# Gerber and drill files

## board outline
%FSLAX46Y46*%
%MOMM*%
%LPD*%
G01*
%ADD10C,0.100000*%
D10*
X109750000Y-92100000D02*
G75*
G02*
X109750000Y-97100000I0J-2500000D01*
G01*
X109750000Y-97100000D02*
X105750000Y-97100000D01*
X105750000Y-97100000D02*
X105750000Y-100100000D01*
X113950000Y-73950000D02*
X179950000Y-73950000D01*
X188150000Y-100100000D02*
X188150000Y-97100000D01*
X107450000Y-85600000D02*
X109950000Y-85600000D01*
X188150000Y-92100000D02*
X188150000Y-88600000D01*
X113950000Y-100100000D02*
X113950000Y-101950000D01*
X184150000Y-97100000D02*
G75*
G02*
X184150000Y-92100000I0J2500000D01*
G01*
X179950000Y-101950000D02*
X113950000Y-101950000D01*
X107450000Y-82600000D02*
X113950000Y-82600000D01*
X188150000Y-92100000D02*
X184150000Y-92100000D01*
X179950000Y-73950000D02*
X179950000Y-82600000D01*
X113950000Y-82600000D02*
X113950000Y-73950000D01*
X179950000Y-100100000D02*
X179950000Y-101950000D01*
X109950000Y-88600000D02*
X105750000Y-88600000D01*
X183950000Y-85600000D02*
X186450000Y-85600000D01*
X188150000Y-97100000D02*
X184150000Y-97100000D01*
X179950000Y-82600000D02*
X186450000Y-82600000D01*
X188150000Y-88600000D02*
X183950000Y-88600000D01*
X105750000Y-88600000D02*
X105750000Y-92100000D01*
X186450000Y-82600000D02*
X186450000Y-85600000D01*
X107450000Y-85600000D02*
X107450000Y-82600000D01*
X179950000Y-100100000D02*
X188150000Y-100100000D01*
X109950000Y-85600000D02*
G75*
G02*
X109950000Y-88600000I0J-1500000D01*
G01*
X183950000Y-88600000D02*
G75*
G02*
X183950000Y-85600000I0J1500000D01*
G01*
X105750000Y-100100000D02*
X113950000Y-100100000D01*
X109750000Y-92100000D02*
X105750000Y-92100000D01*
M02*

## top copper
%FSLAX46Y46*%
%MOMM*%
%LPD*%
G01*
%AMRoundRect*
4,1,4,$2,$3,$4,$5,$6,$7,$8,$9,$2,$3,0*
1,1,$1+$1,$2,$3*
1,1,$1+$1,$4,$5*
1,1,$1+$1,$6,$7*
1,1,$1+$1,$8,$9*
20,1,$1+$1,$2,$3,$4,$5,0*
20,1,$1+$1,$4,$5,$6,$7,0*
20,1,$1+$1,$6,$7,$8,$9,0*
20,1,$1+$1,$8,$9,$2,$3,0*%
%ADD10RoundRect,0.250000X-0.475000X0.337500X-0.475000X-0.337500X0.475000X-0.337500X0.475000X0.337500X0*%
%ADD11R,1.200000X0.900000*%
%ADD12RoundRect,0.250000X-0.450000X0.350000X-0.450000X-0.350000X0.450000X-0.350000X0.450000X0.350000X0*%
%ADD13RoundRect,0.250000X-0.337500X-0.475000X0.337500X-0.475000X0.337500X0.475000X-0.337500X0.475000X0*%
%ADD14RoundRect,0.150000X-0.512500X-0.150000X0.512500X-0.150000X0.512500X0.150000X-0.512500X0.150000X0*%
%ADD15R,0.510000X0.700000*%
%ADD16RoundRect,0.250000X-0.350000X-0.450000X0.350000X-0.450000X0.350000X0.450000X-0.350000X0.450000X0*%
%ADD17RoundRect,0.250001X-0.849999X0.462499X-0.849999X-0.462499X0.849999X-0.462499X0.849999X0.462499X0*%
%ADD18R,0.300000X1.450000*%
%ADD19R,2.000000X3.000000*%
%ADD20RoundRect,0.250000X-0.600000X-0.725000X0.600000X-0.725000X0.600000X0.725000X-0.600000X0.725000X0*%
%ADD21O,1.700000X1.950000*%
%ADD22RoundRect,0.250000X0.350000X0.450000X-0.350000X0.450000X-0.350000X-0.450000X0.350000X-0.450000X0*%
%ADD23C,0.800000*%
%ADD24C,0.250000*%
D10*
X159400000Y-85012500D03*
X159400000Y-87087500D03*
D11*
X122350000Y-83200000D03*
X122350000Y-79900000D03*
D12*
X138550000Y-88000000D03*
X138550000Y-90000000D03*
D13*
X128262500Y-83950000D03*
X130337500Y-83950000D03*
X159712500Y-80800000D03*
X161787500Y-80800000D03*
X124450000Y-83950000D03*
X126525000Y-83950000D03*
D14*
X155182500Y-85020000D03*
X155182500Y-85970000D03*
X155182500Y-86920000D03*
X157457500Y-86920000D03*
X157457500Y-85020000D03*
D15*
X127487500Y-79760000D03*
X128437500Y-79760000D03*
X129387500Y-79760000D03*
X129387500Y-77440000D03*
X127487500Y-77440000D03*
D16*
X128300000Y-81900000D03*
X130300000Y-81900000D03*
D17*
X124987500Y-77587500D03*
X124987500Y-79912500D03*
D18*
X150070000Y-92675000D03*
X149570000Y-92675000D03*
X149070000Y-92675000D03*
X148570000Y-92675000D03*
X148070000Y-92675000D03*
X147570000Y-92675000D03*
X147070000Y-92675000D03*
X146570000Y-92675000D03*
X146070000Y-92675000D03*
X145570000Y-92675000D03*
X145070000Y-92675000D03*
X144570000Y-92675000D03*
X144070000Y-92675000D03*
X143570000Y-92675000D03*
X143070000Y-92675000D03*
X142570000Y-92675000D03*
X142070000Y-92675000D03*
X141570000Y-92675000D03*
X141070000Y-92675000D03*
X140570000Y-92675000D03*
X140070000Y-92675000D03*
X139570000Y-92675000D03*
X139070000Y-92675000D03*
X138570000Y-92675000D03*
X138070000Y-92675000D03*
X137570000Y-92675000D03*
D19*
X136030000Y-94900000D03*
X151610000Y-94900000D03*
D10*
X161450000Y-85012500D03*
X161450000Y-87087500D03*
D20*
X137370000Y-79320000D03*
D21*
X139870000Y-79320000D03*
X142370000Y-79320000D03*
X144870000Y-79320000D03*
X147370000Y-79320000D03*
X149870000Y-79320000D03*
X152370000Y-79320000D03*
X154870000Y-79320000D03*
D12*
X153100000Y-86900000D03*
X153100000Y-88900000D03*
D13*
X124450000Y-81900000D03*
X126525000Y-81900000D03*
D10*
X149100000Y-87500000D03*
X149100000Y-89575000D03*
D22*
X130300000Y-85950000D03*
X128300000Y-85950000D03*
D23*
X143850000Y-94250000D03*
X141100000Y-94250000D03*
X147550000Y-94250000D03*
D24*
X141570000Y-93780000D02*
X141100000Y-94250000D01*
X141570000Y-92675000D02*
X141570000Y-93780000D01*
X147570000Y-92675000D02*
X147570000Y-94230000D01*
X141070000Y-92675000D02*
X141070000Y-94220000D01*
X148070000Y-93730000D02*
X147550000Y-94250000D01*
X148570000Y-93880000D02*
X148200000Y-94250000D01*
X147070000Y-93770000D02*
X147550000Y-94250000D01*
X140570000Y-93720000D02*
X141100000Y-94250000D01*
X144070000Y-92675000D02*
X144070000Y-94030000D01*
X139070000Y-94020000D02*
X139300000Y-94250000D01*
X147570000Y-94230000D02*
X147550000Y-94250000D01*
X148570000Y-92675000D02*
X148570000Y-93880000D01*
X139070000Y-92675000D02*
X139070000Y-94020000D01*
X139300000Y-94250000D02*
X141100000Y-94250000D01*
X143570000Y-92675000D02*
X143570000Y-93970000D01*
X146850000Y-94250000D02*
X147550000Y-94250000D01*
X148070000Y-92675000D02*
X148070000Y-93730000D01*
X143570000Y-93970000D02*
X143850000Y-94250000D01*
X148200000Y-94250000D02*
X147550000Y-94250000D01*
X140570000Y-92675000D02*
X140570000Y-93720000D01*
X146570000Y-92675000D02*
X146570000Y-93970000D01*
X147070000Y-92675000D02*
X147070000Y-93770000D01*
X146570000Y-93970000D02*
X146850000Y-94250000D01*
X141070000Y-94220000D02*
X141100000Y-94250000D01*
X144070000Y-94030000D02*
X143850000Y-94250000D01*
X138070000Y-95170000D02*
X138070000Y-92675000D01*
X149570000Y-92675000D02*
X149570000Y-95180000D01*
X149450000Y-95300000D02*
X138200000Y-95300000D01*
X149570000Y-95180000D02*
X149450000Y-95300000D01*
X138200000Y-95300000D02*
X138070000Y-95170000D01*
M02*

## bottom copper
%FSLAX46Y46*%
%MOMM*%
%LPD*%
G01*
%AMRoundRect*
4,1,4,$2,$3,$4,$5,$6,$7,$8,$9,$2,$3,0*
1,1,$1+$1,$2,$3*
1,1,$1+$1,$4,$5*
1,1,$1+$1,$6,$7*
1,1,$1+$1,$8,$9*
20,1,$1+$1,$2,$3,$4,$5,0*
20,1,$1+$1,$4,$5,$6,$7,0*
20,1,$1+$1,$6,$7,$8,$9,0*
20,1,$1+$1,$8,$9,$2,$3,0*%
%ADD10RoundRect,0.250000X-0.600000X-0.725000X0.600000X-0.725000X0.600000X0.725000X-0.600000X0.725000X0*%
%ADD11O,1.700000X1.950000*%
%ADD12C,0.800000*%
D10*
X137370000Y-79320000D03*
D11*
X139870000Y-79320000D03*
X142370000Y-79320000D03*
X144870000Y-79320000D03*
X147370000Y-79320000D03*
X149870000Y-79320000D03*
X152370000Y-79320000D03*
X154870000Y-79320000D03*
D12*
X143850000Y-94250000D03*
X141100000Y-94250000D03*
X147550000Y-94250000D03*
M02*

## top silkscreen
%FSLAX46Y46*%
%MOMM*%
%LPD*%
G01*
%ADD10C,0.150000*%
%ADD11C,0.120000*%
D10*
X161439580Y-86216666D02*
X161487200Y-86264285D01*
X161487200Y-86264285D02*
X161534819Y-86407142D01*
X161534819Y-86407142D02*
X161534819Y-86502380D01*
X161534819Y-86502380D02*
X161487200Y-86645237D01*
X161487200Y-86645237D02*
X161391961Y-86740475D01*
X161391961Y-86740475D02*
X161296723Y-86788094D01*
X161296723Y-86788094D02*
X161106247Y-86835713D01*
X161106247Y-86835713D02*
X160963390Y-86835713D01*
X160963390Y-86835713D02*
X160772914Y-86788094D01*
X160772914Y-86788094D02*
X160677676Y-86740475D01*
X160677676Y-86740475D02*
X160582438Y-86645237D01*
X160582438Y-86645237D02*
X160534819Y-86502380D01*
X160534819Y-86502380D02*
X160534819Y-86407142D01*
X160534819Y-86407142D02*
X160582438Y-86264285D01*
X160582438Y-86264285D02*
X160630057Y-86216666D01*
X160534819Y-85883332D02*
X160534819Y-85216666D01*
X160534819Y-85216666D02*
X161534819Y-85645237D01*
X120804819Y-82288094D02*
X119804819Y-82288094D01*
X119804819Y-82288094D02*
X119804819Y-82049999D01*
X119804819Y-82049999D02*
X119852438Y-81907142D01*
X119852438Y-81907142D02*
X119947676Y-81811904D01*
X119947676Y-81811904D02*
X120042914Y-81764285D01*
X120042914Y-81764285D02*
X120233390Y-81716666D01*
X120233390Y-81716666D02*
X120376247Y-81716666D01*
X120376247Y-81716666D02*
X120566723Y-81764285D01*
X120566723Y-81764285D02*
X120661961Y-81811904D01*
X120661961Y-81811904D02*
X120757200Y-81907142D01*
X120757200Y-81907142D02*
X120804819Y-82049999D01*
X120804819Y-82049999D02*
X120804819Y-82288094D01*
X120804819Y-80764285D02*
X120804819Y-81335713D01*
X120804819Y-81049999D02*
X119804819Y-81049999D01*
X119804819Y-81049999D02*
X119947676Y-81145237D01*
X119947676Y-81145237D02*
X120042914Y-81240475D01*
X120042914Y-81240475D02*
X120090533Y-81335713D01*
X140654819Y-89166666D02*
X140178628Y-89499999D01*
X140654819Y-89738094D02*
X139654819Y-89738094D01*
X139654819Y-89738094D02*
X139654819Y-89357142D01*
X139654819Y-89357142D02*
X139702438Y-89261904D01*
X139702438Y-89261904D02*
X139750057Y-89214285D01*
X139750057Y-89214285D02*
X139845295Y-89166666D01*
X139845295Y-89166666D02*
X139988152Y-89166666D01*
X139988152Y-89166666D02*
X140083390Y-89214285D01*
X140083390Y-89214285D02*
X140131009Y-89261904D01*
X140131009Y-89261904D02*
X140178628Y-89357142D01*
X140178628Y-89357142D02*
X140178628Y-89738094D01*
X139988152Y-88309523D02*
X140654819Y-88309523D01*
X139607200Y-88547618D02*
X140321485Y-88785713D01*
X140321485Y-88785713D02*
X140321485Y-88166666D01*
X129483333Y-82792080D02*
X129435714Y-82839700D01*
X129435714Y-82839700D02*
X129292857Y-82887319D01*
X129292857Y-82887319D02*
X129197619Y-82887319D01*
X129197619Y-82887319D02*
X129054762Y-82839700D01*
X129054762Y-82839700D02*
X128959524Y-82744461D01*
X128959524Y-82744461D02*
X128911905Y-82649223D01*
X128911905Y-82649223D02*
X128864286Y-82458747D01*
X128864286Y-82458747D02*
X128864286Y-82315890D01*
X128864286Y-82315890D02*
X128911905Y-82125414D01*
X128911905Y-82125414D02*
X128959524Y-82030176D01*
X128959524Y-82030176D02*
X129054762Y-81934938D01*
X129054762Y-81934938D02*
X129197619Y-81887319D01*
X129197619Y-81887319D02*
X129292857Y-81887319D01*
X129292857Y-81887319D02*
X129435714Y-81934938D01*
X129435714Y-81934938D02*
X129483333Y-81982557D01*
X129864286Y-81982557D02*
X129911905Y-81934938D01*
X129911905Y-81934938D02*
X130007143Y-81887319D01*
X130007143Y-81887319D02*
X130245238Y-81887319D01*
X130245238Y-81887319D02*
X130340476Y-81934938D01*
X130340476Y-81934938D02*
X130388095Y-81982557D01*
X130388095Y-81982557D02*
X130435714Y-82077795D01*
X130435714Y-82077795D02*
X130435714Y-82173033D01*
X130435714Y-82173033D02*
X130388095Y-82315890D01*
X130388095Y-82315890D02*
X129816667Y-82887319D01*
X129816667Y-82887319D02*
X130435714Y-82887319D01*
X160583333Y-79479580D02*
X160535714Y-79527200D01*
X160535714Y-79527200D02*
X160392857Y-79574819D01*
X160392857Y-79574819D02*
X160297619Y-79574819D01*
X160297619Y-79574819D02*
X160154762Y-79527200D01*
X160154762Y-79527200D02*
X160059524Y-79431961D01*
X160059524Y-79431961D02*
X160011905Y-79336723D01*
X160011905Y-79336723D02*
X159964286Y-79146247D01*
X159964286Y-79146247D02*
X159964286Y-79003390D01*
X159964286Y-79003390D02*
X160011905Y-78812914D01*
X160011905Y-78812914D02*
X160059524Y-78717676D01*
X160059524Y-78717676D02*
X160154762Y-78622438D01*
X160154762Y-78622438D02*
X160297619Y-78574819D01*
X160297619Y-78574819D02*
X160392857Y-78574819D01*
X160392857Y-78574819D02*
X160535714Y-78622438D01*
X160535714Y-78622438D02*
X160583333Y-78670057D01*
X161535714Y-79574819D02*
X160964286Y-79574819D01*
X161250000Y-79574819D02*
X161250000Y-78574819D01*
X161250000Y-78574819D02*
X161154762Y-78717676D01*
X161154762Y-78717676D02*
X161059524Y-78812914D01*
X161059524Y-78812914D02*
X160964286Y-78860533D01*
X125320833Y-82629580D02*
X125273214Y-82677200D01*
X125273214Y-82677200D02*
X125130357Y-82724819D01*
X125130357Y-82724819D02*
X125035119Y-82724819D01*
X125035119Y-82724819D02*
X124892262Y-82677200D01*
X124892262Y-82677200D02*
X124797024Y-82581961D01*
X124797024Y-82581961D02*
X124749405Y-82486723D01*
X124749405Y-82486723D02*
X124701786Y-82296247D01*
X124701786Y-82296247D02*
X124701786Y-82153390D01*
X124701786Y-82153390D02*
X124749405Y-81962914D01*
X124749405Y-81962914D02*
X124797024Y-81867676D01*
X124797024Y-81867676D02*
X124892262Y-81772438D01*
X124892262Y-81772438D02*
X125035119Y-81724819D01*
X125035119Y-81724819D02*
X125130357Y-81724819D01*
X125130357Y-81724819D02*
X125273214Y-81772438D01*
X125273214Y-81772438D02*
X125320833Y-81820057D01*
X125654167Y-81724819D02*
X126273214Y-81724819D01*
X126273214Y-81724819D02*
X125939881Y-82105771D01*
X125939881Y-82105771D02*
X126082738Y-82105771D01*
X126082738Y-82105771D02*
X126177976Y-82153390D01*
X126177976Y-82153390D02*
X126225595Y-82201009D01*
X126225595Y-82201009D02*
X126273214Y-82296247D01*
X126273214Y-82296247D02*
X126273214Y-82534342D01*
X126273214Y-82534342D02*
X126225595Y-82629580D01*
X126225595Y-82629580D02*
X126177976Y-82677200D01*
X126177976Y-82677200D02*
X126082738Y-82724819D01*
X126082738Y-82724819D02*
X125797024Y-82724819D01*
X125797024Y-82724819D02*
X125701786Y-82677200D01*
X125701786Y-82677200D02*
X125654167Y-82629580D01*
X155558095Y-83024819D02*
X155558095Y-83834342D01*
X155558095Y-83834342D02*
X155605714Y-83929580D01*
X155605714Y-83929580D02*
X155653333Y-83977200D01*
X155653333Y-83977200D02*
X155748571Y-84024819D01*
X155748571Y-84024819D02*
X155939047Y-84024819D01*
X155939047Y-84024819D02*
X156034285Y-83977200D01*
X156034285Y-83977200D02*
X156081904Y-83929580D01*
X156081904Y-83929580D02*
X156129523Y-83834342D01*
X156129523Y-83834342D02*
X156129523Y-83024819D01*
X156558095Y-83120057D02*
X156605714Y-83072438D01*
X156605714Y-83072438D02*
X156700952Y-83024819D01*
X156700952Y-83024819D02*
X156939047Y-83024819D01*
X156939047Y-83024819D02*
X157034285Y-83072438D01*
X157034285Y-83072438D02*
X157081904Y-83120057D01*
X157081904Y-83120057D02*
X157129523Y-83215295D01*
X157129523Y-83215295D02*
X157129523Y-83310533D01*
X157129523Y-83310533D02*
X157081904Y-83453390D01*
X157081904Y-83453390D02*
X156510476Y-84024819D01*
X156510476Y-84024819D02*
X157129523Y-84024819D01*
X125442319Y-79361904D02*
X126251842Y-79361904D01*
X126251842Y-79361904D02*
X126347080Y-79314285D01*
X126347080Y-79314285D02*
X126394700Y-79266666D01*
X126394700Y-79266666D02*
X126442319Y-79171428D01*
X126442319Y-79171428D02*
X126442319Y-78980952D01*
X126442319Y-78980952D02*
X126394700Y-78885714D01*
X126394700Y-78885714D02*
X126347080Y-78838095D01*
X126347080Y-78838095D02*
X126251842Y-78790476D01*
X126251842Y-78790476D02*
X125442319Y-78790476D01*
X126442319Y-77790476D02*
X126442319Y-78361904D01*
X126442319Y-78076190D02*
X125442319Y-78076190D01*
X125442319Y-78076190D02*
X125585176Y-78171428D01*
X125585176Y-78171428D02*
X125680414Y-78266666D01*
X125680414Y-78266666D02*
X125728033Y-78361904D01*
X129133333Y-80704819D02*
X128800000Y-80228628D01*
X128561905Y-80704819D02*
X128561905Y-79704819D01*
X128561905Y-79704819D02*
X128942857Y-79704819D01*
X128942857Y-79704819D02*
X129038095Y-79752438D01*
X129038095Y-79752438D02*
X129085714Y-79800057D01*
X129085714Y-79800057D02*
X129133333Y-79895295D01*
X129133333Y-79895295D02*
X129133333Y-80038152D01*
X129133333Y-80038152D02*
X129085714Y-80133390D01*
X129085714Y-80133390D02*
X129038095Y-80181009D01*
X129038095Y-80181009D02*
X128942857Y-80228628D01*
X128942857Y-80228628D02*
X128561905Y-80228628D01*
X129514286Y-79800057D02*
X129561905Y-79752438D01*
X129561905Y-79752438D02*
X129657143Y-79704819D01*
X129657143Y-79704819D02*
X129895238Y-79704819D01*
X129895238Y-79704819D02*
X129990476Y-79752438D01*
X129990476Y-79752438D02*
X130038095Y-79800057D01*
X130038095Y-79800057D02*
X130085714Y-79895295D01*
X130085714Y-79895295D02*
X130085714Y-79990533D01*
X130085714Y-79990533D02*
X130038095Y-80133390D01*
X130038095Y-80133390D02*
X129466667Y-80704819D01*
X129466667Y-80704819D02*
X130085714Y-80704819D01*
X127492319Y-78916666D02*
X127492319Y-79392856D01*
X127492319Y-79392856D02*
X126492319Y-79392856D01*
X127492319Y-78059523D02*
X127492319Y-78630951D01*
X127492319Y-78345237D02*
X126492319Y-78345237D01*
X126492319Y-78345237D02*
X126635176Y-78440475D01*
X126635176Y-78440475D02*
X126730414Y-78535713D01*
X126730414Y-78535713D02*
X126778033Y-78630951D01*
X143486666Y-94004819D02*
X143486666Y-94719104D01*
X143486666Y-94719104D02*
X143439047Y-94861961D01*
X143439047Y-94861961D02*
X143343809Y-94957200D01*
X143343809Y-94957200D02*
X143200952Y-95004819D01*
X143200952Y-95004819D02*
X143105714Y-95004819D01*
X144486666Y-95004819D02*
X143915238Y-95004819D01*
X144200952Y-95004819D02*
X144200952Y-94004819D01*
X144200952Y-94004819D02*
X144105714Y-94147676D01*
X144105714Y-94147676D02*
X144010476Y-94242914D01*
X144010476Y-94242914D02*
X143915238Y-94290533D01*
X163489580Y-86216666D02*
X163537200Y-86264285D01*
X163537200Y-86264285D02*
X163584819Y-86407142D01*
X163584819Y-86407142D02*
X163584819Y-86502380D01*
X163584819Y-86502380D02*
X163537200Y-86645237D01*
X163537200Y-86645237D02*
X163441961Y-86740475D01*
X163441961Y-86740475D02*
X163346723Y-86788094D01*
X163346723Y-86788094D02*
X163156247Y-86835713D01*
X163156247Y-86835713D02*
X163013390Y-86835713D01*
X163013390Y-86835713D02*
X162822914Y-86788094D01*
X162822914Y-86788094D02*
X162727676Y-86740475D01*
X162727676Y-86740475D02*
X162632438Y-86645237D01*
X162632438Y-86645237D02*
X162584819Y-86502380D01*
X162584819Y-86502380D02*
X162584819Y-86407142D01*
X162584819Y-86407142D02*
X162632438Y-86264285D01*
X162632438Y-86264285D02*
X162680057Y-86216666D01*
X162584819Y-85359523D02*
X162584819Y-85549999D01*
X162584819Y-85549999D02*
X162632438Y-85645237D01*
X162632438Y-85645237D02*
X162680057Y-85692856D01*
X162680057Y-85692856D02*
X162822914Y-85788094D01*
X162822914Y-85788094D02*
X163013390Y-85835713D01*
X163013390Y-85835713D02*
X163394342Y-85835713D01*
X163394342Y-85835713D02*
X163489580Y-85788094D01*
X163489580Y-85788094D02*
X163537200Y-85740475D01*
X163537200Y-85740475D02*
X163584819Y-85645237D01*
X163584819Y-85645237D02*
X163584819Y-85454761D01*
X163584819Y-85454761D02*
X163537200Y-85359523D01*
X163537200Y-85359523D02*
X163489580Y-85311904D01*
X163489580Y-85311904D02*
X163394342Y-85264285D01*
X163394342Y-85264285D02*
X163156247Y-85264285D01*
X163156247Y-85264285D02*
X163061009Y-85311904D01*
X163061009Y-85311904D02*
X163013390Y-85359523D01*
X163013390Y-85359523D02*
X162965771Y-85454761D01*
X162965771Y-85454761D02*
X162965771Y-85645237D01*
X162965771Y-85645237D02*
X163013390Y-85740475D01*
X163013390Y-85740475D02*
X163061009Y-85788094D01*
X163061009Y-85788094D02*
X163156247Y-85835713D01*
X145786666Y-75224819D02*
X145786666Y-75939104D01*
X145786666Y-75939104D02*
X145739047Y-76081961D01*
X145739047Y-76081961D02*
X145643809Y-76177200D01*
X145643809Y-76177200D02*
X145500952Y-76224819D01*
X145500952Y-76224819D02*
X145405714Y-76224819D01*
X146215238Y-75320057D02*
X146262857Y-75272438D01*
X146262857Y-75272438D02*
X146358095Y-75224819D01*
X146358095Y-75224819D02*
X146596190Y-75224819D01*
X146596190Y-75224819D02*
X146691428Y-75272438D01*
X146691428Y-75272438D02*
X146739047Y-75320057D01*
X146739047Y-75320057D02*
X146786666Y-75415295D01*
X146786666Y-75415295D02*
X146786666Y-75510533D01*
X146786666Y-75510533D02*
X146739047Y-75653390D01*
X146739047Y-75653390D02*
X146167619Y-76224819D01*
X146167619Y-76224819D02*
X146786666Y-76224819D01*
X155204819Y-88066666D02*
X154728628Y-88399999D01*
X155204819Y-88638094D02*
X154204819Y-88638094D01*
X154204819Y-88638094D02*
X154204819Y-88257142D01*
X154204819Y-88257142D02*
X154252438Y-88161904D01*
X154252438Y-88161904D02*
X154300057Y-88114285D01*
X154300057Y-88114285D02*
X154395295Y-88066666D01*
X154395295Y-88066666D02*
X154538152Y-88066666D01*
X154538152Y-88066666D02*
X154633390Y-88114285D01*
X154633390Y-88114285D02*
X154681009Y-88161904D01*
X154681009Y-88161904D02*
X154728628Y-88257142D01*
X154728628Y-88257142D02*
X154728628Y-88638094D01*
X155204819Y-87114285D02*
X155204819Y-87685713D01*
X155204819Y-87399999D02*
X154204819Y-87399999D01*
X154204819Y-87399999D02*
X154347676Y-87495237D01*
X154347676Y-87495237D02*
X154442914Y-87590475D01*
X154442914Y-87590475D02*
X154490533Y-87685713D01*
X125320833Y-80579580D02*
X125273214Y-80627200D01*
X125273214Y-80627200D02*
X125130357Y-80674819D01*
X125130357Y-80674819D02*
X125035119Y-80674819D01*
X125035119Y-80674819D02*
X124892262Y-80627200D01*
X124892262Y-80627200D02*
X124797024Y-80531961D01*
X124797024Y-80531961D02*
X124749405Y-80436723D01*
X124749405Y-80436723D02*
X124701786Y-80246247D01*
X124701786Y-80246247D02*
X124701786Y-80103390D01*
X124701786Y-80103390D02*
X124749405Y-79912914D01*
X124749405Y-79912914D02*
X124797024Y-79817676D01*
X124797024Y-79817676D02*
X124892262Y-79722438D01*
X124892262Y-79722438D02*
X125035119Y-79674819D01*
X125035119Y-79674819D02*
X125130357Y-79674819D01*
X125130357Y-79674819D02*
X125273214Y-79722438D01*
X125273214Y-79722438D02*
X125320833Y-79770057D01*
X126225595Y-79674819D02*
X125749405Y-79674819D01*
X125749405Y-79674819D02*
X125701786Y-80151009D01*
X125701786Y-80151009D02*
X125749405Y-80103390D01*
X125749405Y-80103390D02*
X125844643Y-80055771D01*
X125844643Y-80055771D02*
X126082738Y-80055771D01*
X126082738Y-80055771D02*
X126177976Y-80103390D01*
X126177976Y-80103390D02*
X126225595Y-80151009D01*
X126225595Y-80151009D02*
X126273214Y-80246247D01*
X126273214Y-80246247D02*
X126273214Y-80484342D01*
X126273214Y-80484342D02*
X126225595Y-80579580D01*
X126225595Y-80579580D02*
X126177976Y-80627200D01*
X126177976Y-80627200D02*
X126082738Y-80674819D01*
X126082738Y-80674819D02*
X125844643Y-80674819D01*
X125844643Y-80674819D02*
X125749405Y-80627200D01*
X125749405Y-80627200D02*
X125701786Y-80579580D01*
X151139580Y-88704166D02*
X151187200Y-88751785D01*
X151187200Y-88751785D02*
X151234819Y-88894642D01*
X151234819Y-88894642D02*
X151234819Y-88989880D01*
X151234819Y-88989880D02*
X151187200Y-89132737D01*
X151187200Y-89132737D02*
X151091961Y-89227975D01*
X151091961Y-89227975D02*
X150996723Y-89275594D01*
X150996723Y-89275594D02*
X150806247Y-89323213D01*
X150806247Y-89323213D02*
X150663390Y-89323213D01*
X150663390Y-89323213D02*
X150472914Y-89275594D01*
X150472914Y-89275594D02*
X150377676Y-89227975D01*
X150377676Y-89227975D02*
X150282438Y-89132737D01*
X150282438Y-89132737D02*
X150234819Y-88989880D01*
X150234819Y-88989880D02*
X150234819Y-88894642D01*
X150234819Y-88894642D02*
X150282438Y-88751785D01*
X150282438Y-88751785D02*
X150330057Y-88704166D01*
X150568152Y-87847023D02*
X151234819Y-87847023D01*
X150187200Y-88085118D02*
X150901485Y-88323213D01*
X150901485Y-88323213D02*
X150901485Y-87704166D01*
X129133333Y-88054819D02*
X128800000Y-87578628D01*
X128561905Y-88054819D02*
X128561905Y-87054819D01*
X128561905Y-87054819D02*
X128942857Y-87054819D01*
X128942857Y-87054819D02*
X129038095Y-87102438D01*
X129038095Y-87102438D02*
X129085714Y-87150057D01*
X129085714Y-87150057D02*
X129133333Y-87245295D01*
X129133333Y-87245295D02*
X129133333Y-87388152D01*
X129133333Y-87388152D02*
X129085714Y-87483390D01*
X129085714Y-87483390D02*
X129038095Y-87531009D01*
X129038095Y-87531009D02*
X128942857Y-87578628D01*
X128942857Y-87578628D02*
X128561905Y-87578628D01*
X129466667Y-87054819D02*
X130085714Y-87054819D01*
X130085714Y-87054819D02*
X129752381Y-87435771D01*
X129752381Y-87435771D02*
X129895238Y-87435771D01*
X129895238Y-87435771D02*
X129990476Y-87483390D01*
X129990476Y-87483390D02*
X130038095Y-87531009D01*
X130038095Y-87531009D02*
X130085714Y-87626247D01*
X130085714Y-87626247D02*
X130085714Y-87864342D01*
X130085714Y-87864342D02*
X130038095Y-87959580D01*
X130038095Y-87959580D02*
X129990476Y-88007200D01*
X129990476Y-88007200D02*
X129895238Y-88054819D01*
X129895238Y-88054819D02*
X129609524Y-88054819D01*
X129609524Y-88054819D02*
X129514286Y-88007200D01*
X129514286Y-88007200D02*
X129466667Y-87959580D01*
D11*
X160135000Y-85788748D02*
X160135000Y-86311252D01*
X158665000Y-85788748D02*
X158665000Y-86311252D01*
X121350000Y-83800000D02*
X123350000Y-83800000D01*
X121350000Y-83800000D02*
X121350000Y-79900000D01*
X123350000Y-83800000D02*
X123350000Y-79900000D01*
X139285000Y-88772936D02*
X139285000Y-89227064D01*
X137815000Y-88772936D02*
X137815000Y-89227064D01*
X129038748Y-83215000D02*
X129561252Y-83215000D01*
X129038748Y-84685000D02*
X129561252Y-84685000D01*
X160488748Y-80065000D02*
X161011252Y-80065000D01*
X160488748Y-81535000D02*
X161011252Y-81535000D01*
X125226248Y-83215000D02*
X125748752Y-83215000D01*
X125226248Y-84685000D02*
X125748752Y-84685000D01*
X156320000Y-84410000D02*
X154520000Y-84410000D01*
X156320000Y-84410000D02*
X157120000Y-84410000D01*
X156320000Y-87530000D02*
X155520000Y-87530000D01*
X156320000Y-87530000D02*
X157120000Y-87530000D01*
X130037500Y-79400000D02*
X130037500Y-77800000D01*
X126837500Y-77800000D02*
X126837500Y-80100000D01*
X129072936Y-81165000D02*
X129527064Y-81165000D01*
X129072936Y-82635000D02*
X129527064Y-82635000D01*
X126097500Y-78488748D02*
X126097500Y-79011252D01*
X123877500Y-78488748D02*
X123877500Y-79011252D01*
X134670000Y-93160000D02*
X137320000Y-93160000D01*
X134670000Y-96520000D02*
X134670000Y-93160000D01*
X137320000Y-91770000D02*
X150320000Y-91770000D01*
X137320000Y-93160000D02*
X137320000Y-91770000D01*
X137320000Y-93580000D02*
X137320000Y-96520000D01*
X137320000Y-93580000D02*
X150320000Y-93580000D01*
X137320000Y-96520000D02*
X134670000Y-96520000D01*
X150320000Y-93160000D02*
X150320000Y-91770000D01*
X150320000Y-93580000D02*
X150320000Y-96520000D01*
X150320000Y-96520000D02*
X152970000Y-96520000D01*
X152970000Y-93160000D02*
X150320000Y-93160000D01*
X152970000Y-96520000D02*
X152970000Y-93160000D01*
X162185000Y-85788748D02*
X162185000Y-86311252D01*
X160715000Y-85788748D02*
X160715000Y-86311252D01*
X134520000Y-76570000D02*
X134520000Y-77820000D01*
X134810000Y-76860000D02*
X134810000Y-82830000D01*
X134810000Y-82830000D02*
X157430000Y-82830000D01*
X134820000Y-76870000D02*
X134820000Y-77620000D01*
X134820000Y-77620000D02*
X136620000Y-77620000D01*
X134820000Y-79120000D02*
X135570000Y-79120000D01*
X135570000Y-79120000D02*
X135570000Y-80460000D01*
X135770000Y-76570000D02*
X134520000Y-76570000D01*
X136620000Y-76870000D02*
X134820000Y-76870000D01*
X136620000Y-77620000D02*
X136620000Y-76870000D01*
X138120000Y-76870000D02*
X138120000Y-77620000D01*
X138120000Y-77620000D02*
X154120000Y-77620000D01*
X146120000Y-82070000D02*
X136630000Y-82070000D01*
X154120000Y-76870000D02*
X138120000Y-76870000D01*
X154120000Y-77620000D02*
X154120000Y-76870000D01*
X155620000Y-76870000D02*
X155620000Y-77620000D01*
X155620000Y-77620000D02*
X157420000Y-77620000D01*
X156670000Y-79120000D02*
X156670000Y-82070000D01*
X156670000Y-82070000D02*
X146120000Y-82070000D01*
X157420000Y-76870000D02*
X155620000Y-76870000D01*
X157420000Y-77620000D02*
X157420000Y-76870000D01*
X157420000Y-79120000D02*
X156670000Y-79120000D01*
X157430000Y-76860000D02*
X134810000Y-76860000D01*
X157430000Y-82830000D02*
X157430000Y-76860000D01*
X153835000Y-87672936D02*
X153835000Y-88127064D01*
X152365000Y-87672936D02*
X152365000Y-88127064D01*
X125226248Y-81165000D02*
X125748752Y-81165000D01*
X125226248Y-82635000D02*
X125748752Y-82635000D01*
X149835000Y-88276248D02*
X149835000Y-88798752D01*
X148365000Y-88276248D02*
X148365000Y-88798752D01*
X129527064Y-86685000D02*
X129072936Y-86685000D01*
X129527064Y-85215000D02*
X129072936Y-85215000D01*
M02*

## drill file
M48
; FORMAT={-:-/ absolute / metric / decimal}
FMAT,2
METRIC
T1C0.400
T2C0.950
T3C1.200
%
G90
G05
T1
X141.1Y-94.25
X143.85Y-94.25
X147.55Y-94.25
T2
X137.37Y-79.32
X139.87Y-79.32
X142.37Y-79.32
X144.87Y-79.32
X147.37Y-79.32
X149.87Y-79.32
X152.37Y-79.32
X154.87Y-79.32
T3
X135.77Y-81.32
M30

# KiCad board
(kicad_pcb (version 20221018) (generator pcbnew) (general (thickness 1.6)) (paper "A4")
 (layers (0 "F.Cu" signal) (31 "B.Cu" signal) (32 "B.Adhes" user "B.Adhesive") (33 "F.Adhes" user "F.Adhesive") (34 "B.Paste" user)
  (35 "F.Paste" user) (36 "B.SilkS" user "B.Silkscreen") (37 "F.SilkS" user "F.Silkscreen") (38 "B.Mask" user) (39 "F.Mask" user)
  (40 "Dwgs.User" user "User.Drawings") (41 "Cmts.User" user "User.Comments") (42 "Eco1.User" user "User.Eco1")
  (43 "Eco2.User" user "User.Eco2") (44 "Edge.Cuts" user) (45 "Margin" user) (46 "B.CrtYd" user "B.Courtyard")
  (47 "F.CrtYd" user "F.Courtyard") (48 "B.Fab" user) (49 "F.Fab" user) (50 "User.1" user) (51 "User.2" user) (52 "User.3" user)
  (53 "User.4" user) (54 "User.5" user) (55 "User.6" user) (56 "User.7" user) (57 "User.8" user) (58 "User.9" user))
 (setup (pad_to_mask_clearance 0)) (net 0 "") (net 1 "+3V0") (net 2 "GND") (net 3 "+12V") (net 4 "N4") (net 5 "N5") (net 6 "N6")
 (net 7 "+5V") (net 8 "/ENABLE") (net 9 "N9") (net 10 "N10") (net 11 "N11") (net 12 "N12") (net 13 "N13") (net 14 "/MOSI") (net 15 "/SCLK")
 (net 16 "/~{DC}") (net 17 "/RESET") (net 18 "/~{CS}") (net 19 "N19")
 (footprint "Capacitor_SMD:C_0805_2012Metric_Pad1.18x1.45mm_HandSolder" (layer "F.Cu") (at 159.4 86.05 -90)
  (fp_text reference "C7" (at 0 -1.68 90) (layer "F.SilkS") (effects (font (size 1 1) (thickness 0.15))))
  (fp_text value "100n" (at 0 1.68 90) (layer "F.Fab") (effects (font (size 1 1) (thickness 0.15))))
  (fp_line (start -0.261252 -0.735) (end 0.261252 -0.735) (stroke (width 0.12) (type solid)) (layer "F.SilkS"))
  (fp_line (start -0.261252 0.735) (end 0.261252 0.735) (stroke (width 0.12) (type solid)) (layer "F.SilkS"))
  (pad "1" smd roundrect (at -1.0375 0 270) (size 1.175 1.45) (layers "F.Cu" "F.Paste" "F.Mask") (roundrect_rratio 0.212766) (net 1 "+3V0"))
  (pad "2" smd roundrect (at 1.0375 0 270) (size 1.175 1.45) (layers "F.Cu" "F.Paste" "F.Mask") (roundrect_rratio 0.212766) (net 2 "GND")))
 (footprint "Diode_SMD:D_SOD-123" (layer "F.Cu") (at 122.35 81.55 90)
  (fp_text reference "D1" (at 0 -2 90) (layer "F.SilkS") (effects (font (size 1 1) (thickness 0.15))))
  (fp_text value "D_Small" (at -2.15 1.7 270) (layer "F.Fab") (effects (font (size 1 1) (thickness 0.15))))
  (fp_line (start -2.25 -1) (end -2.25 1) (stroke (width 0.12) (type solid)) (layer "F.SilkS"))
  (fp_line (start -2.25 -1) (end 1.65 -1) (stroke (width 0.12) (type solid)) (layer "F.SilkS"))
  (fp_line (start -2.25 1) (end 1.65 1) (stroke (width 0.12) (type solid)) (layer "F.SilkS"))
  (pad "1" smd rect (at -1.65 0 90) (size 0.9 1.2) (layers "F.Cu" "F.Paste" "F.Mask") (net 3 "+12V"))
  (pad "2" smd rect (at 1.65 0 90) (size 0.9 1.2) (layers "F.Cu" "F.Paste" "F.Mask") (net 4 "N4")))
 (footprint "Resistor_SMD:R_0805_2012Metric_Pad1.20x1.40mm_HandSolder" (layer "F.Cu") (at 138.55 89 -90)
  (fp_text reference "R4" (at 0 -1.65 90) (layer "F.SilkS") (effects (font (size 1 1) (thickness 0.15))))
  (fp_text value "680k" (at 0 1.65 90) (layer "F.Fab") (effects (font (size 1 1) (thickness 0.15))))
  (fp_line (start -0.227064 -0.735) (end 0.227064 -0.735) (stroke (width 0.12) (type solid)) (layer "F.SilkS"))
  (fp_line (start -0.227064 0.735) (end 0.227064 0.735) (stroke (width 0.12) (type solid)) (layer "F.SilkS"))
  (pad "1" smd roundrect (at -1 0 270) (size 1.2 1.4) (layers "F.Cu" "F.Paste" "F.Mask") (roundrect_rratio 0.208333) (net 2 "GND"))
  (pad "2" smd roundrect (at 1 0 270) (size 1.2 1.4) (layers "F.Cu" "F.Paste" "F.Mask") (roundrect_rratio 0.208333) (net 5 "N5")))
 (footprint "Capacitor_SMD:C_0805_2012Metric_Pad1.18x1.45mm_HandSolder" (layer "F.Cu") (at 129.3 83.95)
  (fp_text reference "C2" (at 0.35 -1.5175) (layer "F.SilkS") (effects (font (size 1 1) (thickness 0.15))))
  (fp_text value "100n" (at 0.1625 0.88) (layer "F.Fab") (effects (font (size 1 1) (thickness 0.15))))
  (fp_line (start -0.261252 -0.735) (end 0.261252 -0.735) (stroke (width 0.12) (type solid)) (layer "F.SilkS"))
  (fp_line (start -0.261252 0.735) (end 0.261252 0.735) (stroke (width 0.12) (type solid)) (layer "F.SilkS"))
  (pad "1" smd roundrect (at -1.0375 0) (size 1.175 1.45) (layers "F.Cu" "F.Paste" "F.Mask") (roundrect_rratio 0.212766) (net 4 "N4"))
  (pad "2" smd roundrect (at 1.0375 0) (size 1.175 1.45) (layers "F.Cu" "F.Paste" "F.Mask") (roundrect_rratio 0.212766) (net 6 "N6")))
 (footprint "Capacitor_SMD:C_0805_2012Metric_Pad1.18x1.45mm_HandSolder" (layer "F.Cu") (at 160.75 80.8)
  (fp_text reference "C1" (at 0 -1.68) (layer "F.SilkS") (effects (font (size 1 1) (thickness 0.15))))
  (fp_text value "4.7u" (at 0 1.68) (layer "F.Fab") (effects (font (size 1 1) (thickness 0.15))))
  (fp_line (start -0.261252 -0.735) (end 0.261252 -0.735) (stroke (width 0.12) (type solid)) (layer "F.SilkS"))
  (fp_line (start -0.261252 0.735) (end 0.261252 0.735) (stroke (width 0.12) (type solid)) (layer "F.SilkS"))
  (pad "1" smd roundrect (at -1.0375 0) (size 1.175 1.45) (layers "F.Cu" "F.Paste" "F.Mask") (roundrect_rratio 0.212766) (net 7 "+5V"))
  (pad "2" smd roundrect (at 1.0375 0) (size 1.175 1.45) (layers "F.Cu" "F.Paste" "F.Mask") (roundrect_rratio 0.212766) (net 2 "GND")))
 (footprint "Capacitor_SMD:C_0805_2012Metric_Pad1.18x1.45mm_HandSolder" (layer "F.Cu") (at 125.4875 83.95)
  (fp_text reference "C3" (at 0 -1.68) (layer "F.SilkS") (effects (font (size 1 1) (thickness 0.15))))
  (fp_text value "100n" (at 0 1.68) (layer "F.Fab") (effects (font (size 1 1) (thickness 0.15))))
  (fp_line (start -0.261252 -0.735) (end 0.261252 -0.735) (stroke (width 0.12) (type solid)) (layer "F.SilkS"))
  (fp_line (start -0.261252 0.735) (end 0.261252 0.735) (stroke (width 0.12) (type solid)) (layer "F.SilkS"))
  (pad "1" smd roundrect (at -1.0375 0) (size 1.175 1.45) (layers "F.Cu" "F.Paste" "F.Mask") (roundrect_rratio 0.212766) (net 3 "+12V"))
  (pad "2" smd roundrect (at 1.0375 0) (size 1.175 1.45) (layers "F.Cu" "F.Paste" "F.Mask") (roundrect_rratio 0.212766) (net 2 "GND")))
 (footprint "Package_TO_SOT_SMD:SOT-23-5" (layer "F.Cu") (at 156.32 85.97)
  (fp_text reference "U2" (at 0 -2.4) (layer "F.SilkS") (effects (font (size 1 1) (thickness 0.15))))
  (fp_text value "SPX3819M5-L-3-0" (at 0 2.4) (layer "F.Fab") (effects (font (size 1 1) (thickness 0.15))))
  (fp_line (start 0 -1.56) (end -1.8 -1.56) (stroke (width 0.12) (type solid)) (layer "F.SilkS"))
  (fp_line (start 0 -1.56) (end 0.8 -1.56) (stroke (width 0.12) (type solid)) (layer "F.SilkS"))
  (fp_line (start 0 1.56) (end -0.8 1.56) (stroke (width 0.12) (type solid)) (layer "F.SilkS"))
  (fp_line (start 0 1.56) (end 0.8 1.56) (stroke (width 0.12) (type solid)) (layer "F.SilkS"))
  (pad "1" smd roundrect (at -1.1375 -0.95) (size 1.325 0.6) (layers "F.Cu" "F.Paste" "F.Mask") (roundrect_rratio 0.25) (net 7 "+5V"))
  (pad "2" smd roundrect (at -1.1375 0) (size 1.325 0.6) (layers "F.Cu" "F.Paste" "F.Mask") (roundrect_rratio 0.25) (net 2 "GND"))
  (pad "3" smd roundrect (at -1.1375 0.95) (size 1.325 0.6) (layers "F.Cu" "F.Paste" "F.Mask") (roundrect_rratio 0.25) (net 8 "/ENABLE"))
  (pad "4" smd roundrect (at 1.1375 0.95) (size 1.325 0.6) (layers "F.Cu" "F.Paste" "F.Mask") (roundrect_rratio 0.25) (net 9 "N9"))
  (pad "5" smd roundrect (at 1.1375 -0.95) (size 1.325 0.6) (layers "F.Cu" "F.Paste" "F.Mask") (roundrect_rratio 0.25) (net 1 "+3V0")))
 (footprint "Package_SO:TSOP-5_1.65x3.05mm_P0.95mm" (layer "F.Cu") (at 128.4375 78.6 90)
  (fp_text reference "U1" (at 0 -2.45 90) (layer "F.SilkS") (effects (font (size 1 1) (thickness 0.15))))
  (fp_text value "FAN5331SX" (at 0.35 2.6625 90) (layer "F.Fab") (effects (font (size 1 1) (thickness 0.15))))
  (fp_line (start -0.8 1.6) (end 0.8 1.6) (stroke (width 0.12) (type solid)) (layer "F.SilkS"))
  (fp_line (start 0.8 -1.6) (end -1.5 -1.6) (stroke (width 0.12) (type solid)) (layer "F.SilkS"))
  (pad "1" smd rect (at -1.16 -0.95 90) (size 0.7 0.51) (layers "F.Cu" "F.Paste" "F.Mask") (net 4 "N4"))
  (pad "2" smd rect (at -1.16 0 90) (size 0.7 0.51) (layers "F.Cu" "F.Paste" "F.Mask") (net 2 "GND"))
  (pad "3" smd rect (at -1.16 0.95 90) (size 0.7 0.51) (layers "F.Cu" "F.Paste" "F.Mask") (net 6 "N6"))
  (pad "4" smd rect (at 1.16 0.95 90) (size 0.7 0.51) (layers "F.Cu" "F.Paste" "F.Mask") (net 8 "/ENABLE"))
  (pad "5" smd rect (at 1.16 -0.95 90) (size 0.7 0.51) (layers "F.Cu" "F.Paste" "F.Mask") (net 7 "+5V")))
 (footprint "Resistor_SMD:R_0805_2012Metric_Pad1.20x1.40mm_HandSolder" (layer "F.Cu") (at 129.3 81.9)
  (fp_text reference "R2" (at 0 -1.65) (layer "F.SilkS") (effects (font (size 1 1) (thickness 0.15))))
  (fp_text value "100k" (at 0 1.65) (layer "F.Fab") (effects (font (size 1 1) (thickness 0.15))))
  (fp_line (start -0.227064 -0.735) (end 0.227064 -0.735) (stroke (width 0.12) (type solid)) (layer "F.SilkS"))
  (fp_line (start -0.227064 0.735) (end 0.227064 0.735) (stroke (width 0.12) (type solid)) (layer "F.SilkS"))
  (pad "1" smd roundrect (at -1 0) (size 1.2 1.4) (layers "F.Cu" "F.Paste" "F.Mask") (roundrect_rratio 0.208333) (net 4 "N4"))
  (pad "2" smd roundrect (at 1 0) (size 1.2 1.4) (layers "F.Cu" "F.Paste" "F.Mask") (roundrect_rratio 0.208333) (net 6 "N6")))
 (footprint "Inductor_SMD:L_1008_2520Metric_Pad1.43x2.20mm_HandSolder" (layer "F.Cu") (at 124.9875 78.75 -90)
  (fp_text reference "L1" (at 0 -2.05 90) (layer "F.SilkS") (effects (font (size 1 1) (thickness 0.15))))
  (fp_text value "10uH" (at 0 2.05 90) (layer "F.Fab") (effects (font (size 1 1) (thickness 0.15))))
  (fp_line (start -0.261252 -1.11) (end 0.261252 -1.11) (stroke (width 0.12) (type solid)) (layer "F.SilkS"))
  (fp_line (start -0.261252 1.11) (end 0.261252 1.11) (stroke (width 0.12) (type solid)) (layer "F.SilkS"))
  (pad "1" smd roundrect (at -1.1625 0 270) (size 1.425 2.2) (layers "F.Cu" "F.Paste" "F.Mask") (roundrect_rratio 0.175439) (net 7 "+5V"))
  (pad "2" smd roundrect (at 1.1625 0 270) (size 1.425 2.2) (layers "F.Cu" "F.Paste" "F.Mask") (roundrect_rratio 0.175439) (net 4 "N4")))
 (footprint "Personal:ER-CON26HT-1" (layer "F.Cu") (at 143.82 92.675)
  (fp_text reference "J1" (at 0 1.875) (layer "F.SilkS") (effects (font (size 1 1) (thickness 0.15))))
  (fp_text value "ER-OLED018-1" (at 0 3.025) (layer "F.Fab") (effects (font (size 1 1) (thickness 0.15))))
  (fp_line (start -9.15 0.485) (end -6.5 0.485) (stroke (width 0.12) (type solid)) (layer "F.SilkS"))
  (fp_line (start -9.15 3.845) (end -9.15 0.485) (stroke (width 0.12) (type solid)) (layer "F.SilkS"))
  (fp_line (start -6.5 -0.905) (end 6.5 -0.905) (stroke (width 0.12) (type solid)) (layer "F.SilkS"))
  (fp_line (start -6.5 0.485) (end -6.5 -0.905) (stroke (width 0.12) (type solid)) (layer "F.SilkS"))
  (fp_line (start -6.5 0.905) (end -6.5 3.845) (stroke (width 0.12) (type solid)) (layer "F.SilkS"))
  (fp_line (start -6.5 0.905) (end 6.5 0.905) (stroke (width 0.12) (type solid)) (layer "F.SilkS"))
  (fp_line (start -6.5 3.845) (end -9.15 3.845) (stroke (width 0.12) (type solid)) (layer "F.SilkS"))
  (fp_line (start 6.5 0.485) (end 6.5 -0.905) (stroke (width 0.12) (type solid)) (layer "F.SilkS"))
  (fp_line (start 6.5 0.905) (end 6.5 3.845) (stroke (width 0.12) (type solid)) (layer "F.SilkS"))
  (fp_line (start 6.5 3.845) (end 9.15 3.845) (stroke (width 0.12) (type solid)) (layer "F.SilkS"))
  (fp_line (start 9.15 0.485) (end 6.5 0.485) (stroke (width 0.12) (type solid)) (layer "F.SilkS"))
  (fp_line (start 9.15 3.845) (end 9.15 0.485) (stroke (width 0.12) (type solid)) (layer "F.SilkS"))
  (pad "1" smd rect (at 6.25 0) (size 0.3 1.45) (layers "F.Cu" "F.Paste" "F.Mask") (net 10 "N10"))
  (pad "2" smd rect (at 5.75 0) (size 0.3 1.45) (layers "F.Cu" "F.Paste" "F.Mask") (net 3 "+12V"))
  (pad "3" smd rect (at 5.25 0) (size 0.3 1.45) (layers "F.Cu" "F.Paste" "F.Mask") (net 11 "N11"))
  (pad "4" smd rect (at 4.75 0) (size 0.3 1.45) (layers "F.Cu" "F.Paste" "F.Mask") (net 2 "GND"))
  (pad "5" smd rect (at 4.25 0) (size 0.3 1.45) (layers "F.Cu" "F.Paste" "F.Mask") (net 2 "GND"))
  (pad "6" smd rect (at 3.75 0) (size 0.3 1.45) (layers "F.Cu" "F.Paste" "F.Mask") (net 2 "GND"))
  (pad "7" smd rect (at 3.25 0) (size 0.3 1.45) (layers "F.Cu" "F.Paste" "F.Mask") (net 2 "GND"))
  (pad "8" smd rect (at 2.75 0) (size 0.3 1.45) (layers "F.Cu" "F.Paste" "F.Mask") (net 2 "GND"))
  (pad "9" smd rect (at 2.25 0) (size 0.3 1.45) (layers "F.Cu" "F.Paste" "F.Mask") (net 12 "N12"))
  (pad "10" smd rect (at 1.75 0) (size 0.3 1.45) (layers "F.Cu" "F.Paste" "F.Mask") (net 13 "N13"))
  (pad "11" smd rect (at 1.25 0) (size 0.3 1.45) (layers "F.Cu" "F.Paste" "F.Mask") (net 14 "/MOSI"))
  (pad "12" smd rect (at 0.75 0) (size 0.3 1.45) (layers "F.Cu" "F.Paste" "F.Mask") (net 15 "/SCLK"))
  (pad "13" smd rect (at 0.25 0) (size 0.3 1.45) (layers "F.Cu" "F.Paste" "F.Mask") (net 2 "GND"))
  (pad "14" smd rect (at -0.25 0) (size 0.3 1.45) (layers "F.Cu" "F.Paste" "F.Mask") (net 2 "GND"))
  (pad "15" smd rect (at -0.75 0) (size 0.3 1.45) (layers "F.Cu" "F.Paste" "F.Mask") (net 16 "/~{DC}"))
  (pad "16" smd rect (at -1.25 0) (size 0.3 1.45) (layers "F.Cu" "F.Paste" "F.Mask") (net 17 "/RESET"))
  (pad "17" smd rect (at -1.75 0) (size 0.3 1.45) (layers "F.Cu" "F.Paste" "F.Mask") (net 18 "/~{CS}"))
  (pad "18" smd rect (at -2.25 0) (size 0.3 1.45) (layers "F.Cu" "F.Paste" "F.Mask") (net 2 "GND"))
  (pad "19" smd rect (at -2.75 0) (size 0.3 1.45) (layers "F.Cu" "F.Paste" "F.Mask") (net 2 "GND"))
  (pad "20" smd rect (at -3.25 0) (size 0.3 1.45) (layers "F.Cu" "F.Paste" "F.Mask") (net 2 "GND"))
  (pad "21" smd rect (at -3.75 0) (size 0.3 1.45) (layers "F.Cu" "F.Paste" "F.Mask") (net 1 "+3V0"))
  (pad "22" smd rect (at -4.25 0) (size 0.3 1.45) (layers "F.Cu" "F.Paste" "F.Mask") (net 1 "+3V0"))
  (pad "23" smd rect (at -4.75 0) (size 0.3 1.45) (layers "F.Cu" "F.Paste" "F.Mask") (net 2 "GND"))
  (pad "24" smd rect (at -5.25 0) (size 0.3 1.45) (layers "F.Cu" "F.Paste" "F.Mask") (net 5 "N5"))
  (pad "25" smd rect (at -5.75 0) (size 0.3 1.45) (layers "F.Cu" "F.Paste" "F.Mask") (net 3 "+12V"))
  (pad "26" smd rect (at -6.25 0) (size 0.3 1.45) (layers "F.Cu" "F.Paste" "F.Mask") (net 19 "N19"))
  (pad "MT" smd rect (at -7.79 2.225) (size 2 3) (layers "F.Cu" "F.Paste" "F.Mask"))
  (pad "MT" smd rect (at 7.79 2.225) (size 2 3) (layers "F.Cu" "F.Paste" "F.Mask")))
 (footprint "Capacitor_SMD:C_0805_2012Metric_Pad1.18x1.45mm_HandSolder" (layer "F.Cu") (at 161.45 86.05 -90)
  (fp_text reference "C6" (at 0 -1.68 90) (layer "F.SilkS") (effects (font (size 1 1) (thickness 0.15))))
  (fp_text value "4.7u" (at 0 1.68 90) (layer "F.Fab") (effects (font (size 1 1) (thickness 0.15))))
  (fp_line (start -0.261252 -0.735) (end 0.261252 -0.735) (stroke (width 0.12) (type solid)) (layer "F.SilkS"))
  (fp_line (start -0.261252 0.735) (end 0.261252 0.735) (stroke (width 0.12) (type solid)) (layer "F.SilkS"))
  (pad "1" smd roundrect (at -1.0375 0 270) (size 1.175 1.45) (layers "F.Cu" "F.Paste" "F.Mask") (roundrect_rratio 0.212766) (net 1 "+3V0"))
  (pad "2" smd roundrect (at 1.0375 0 270) (size 1.175 1.45) (layers "F.Cu" "F.Paste" "F.Mask") (roundrect_rratio 0.212766) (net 2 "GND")))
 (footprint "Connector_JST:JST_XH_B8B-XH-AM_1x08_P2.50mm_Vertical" (layer "F.Cu") (at 137.37 79.32)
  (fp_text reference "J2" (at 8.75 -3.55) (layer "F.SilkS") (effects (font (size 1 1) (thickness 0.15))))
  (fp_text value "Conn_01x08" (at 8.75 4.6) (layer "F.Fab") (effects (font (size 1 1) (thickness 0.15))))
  (fp_line (start -2.85 -2.75) (end -2.85 -1.5) (stroke (width 0.12) (type solid)) (layer "F.SilkS"))
  (fp_line (start -2.56 -2.46) (end -2.56 3.51) (stroke (width 0.12) (type solid)) (layer "F.SilkS"))
  (fp_line (start -2.56 3.51) (end 20.06 3.51) (stroke (width 0.12) (type solid)) (layer "F.SilkS"))
  (fp_line (start -2.55 -2.45) (end -2.55 -1.7) (stroke (width 0.12) (type solid)) (layer "F.SilkS"))
  (fp_line (start -2.55 -1.7) (end -0.75 -1.7) (stroke (width 0.12) (type solid)) (layer "F.SilkS"))
  (fp_line (start -2.55 -0.2) (end -1.8 -0.2) (stroke (width 0.12) (type solid)) (layer "F.SilkS"))
  (fp_line (start -1.8 -0.2) (end -1.8 1.14) (stroke (width 0.12) (type solid)) (layer "F.SilkS"))
  (fp_line (start -1.6 -2.75) (end -2.85 -2.75) (stroke (width 0.12) (type solid)) (layer "F.SilkS"))
  (fp_line (start -0.75 -2.45) (end -2.55 -2.45) (stroke (width 0.12) (type solid)) (layer "F.SilkS"))
  (fp_line (start -0.75 -1.7) (end -0.75 -2.45) (stroke (width 0.12) (type solid)) (layer "F.SilkS"))
  (fp_line (start 0.75 -2.45) (end 0.75 -1.7) (stroke (width 0.12) (type solid)) (layer "F.SilkS"))
  (fp_line (start 0.75 -1.7) (end 16.75 -1.7) (stroke (width 0.12) (type solid)) (layer "F.SilkS"))
  (fp_line (start 8.75 2.75) (end -0.74 2.75) (stroke (width 0.12) (type solid)) (layer "F.SilkS"))
  (fp_line (start 16.75 -2.45) (end 0.75 -2.45) (stroke (width 0.12) (type solid)) (layer "F.SilkS"))
  (fp_line (start 16.75 -1.7) (end 16.75 -2.45) (stroke (width 0.12) (type solid)) (layer "F.SilkS"))
  (fp_line (start 18.25 -2.45) (end 18.25 -1.7) (stroke (width 0.12) (type solid)) (layer "F.SilkS"))
  (fp_line (start 18.25 -1.7) (end 20.05 -1.7) (stroke (width 0.12) (type solid)) (layer "F.SilkS"))
  (fp_line (start 19.3 -0.2) (end 19.3 2.75) (stroke (width 0.12) (type solid)) (layer "F.SilkS"))
  (fp_line (start 19.3 2.75) (end 8.75 2.75) (stroke (width 0.12) (type solid)) (layer "F.SilkS"))
  (fp_line (start 20.05 -2.45) (end 18.25 -2.45) (stroke (width 0.12) (type solid)) (layer "F.SilkS"))
  (fp_line (start 20.05 -1.7) (end 20.05 -2.45) (stroke (width 0.12) (type solid)) (layer "F.SilkS"))
  (fp_line (start 20.05 -0.2) (end 19.3 -0.2) (stroke (width 0.12) (type solid)) (layer "F.SilkS"))
  (fp_line (start 20.06 -2.46) (end -2.56 -2.46) (stroke (width 0.12) (type solid)) (layer "F.SilkS"))
  (fp_line (start 20.06 3.51) (end 20.06 -2.46) (stroke (width 0.12) (type solid)) (layer "F.SilkS"))
  (pad "" np_thru_hole circle (at -1.6 2) (size 1.2 1.2) (drill 1.2) (layers "*.Cu" "*.Mask"))
  (pad "1" thru_hole roundrect (at 0 0) (size 1.7 1.95) (drill 0.95) (layers "*.Cu" "*.Mask") (roundrect_rratio 0.147059) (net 7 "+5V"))
  (pad "2" thru_hole oval (at 2.5 0) (size 1.7 1.95) (drill 0.95) (layers "*.Cu" "*.Mask") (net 8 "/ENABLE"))
  (pad "3" thru_hole oval (at 5 0) (size 1.7 1.95) (drill 0.95) (layers "*.Cu" "*.Mask") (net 18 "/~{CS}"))
  (pad "4" thru_hole oval (at 7.5 0) (size 1.7 1.95) (drill 0.95) (layers "*.Cu" "*.Mask") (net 17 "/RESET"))
  (pad "5" thru_hole oval (at 10 0) (size 1.7 1.95) (drill 0.95) (layers "*.Cu" "*.Mask") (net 16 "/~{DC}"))
  (pad "6" thru_hole oval (at 12.5 0) (size 1.7 1.95) (drill 0.95) (layers "*.Cu" "*.Mask") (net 15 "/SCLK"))
  (pad "7" thru_hole oval (at 15 0) (size 1.7 1.95) (drill 0.95) (layers "*.Cu" "*.Mask") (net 14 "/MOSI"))
  (pad "8" thru_hole oval (at 17.5 0) (size 1.7 1.95) (drill 0.95) (layers "*.Cu" "*.Mask") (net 2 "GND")))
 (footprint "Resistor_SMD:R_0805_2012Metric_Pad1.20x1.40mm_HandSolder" (layer "F.Cu") (at 153.1 87.9 -90)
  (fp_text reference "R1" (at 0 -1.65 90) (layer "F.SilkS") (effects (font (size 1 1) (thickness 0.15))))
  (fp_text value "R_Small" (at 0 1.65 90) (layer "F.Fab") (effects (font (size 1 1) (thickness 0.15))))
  (fp_line (start -0.227064 -0.735) (end 0.227064 -0.735) (stroke (width 0.12) (type solid)) (layer "F.SilkS"))
  (fp_line (start -0.227064 0.735) (end 0.227064 0.735) (stroke (width 0.12) (type solid)) (layer "F.SilkS"))
  (pad "1" smd roundrect (at -1 0 270) (size 1.2 1.4) (layers "F.Cu" "F.Paste" "F.Mask") (roundrect_rratio 0.208333) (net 8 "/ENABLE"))
  (pad "2" smd roundrect (at 1 0 270) (size 1.2 1.4) (layers "F.Cu" "F.Paste" "F.Mask") (roundrect_rratio 0.208333) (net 2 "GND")))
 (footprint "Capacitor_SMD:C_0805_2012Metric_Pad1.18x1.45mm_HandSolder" (layer "F.Cu") (at 125.4875 81.9)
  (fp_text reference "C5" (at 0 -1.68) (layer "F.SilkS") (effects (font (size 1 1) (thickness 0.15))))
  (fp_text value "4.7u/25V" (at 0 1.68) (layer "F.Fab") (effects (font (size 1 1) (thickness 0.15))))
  (fp_line (start -0.261252 -0.735) (end 0.261252 -0.735) (stroke (width 0.12) (type solid)) (layer "F.SilkS"))
  (fp_line (start -0.261252 0.735) (end 0.261252 0.735) (stroke (width 0.12) (type solid)) (layer "F.SilkS"))
  (pad "1" smd roundrect (at -1.0375 0) (size 1.175 1.45) (layers "F.Cu" "F.Paste" "F.Mask") (roundrect_rratio 0.212766) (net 3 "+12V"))
  (pad "2" smd roundrect (at 1.0375 0) (size 1.175 1.45) (layers "F.Cu" "F.Paste" "F.Mask") (roundrect_rratio 0.212766) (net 2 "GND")))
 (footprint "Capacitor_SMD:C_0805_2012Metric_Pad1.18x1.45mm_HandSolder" (layer "F.Cu") (at 149.1 88.5375 -90)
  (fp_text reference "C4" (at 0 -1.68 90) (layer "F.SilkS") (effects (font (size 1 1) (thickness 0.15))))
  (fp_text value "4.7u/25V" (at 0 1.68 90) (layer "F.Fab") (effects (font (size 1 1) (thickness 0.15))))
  (fp_line (start -0.261252 -0.735) (end 0.261252 -0.735) (stroke (width 0.12) (type solid)) (layer "F.SilkS"))
  (fp_line (start -0.261252 0.735) (end 0.261252 0.735) (stroke (width 0.12) (type solid)) (layer "F.SilkS"))
  (pad "1" smd roundrect (at -1.0375 0 270) (size 1.175 1.45) (layers "F.Cu" "F.Paste" "F.Mask") (roundrect_rratio 0.212766) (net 2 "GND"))
  (pad "2" smd roundrect (at 1.0375 0 270) (size 1.175 1.45) (layers "F.Cu" "F.Paste" "F.Mask") (roundrect_rratio 0.212766) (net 11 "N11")))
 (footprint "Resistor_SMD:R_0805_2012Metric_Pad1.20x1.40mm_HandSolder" (layer "F.Cu") (at 129.3 85.95 180)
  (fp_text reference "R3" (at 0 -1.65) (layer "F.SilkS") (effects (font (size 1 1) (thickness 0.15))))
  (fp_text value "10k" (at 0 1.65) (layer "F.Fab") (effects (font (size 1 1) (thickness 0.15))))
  (fp_line (start -0.227064 -0.735) (end 0.227064 -0.735) (stroke (width 0.12) (type solid)) (layer "F.SilkS"))
  (fp_line (start -0.227064 0.735) (end 0.227064 0.735) (stroke (width 0.12) (type solid)) (layer "F.SilkS"))
  (pad "1" smd roundrect (at -1 0 180) (size 1.2 1.4) (layers "F.Cu" "F.Paste" "F.Mask") (roundrect_rratio 0.208333) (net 6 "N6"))
  (pad "2" smd roundrect (at 1 0 180) (size 1.2 1.4) (layers "F.Cu" "F.Paste" "F.Mask") (roundrect_rratio 0.208333) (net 2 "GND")))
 (gr_arc (start 109.75 92.1) (mid 112.25 94.6) (end 109.75 97.1) (stroke (width 0.1) (type solid)) (layer "Edge.Cuts"))
 (gr_line (start 109.75 97.1) (end 105.75 97.1) (stroke (width 0.1) (type solid)) (layer "Edge.Cuts"))
 (gr_line (start 105.75 97.1) (end 105.75 100.1) (stroke (width 0.1) (type solid)) (layer "Edge.Cuts"))
 (gr_line (start 113.95 73.95) (end 179.95 73.95) (stroke (width 0.1) (type solid)) (layer "Edge.Cuts"))
 (gr_line (start 188.15 100.1) (end 188.15 97.1) (stroke (width 0.1) (type solid)) (layer "Edge.Cuts"))
 (gr_line (start 107.45 85.6) (end 109.95 85.6) (stroke (width 0.1) (type solid)) (layer "Edge.Cuts"))
 (gr_line (start 188.15 92.1) (end 188.15 88.6) (stroke (width 0.1) (type solid)) (layer "Edge.Cuts"))
 (gr_line (start 113.95 100.1) (end 113.95 101.95) (stroke (width 0.1) (type solid)) (layer "Edge.Cuts"))
 (gr_arc (start 184.15 97.1) (mid 181.65 94.6) (end 184.15 92.1) (stroke (width 0.1) (type solid)) (layer "Edge.Cuts"))
 (gr_line (start 179.95 101.95) (end 113.95 101.95) (stroke (width 0.1) (type solid)) (layer "Edge.Cuts"))
 (gr_line (start 107.45 82.6) (end 113.95 82.6) (stroke (width 0.1) (type solid)) (layer "Edge.Cuts"))
 (gr_line (start 188.15 92.1) (end 184.15 92.1) (stroke (width 0.1) (type solid)) (layer "Edge.Cuts"))
 (gr_line (start 179.95 73.95) (end 179.95 82.6) (stroke (width 0.1) (type solid)) (layer "Edge.Cuts"))
 (gr_line (start 113.95 82.6) (end 113.95 73.95) (stroke (width 0.1) (type solid)) (layer "Edge.Cuts"))
 (gr_line (start 179.95 100.1) (end 179.95 101.95) (stroke (width 0.1) (type solid)) (layer "Edge.Cuts"))
 (gr_line (start 109.95 88.6) (end 105.75 88.6) (stroke (width 0.1) (type solid)) (layer "Edge.Cuts"))
 (gr_line (start 183.95 85.6) (end 186.45 85.6) (stroke (width 0.1) (type solid)) (layer "Edge.Cuts"))
 (gr_line (start 188.15 97.1) (end 184.15 97.1) (stroke (width 0.1) (type solid)) (layer "Edge.Cuts"))
 (gr_line (start 179.95 82.6) (end 186.45 82.6) (stroke (width 0.1) (type solid)) (layer "Edge.Cuts"))
 (gr_line (start 188.15 88.6) (end 183.95 88.6) (stroke (width 0.1) (type solid)) (layer "Edge.Cuts"))
 (gr_line (start 105.75 88.6) (end 105.75 92.1) (stroke (width 0.1) (type solid)) (layer "Edge.Cuts"))
 (gr_line (start 186.45 82.6) (end 186.45 85.6) (stroke (width 0.1) (type solid)) (layer "Edge.Cuts"))
 (gr_line (start 107.45 85.6) (end 107.45 82.6) (stroke (width 0.1) (type solid)) (layer "Edge.Cuts"))
 (gr_line (start 179.95 100.1) (end 188.15 100.1) (stroke (width 0.1) (type solid)) (layer "Edge.Cuts"))
 (gr_arc (start 109.95 85.6) (mid 111.45 87.1) (end 109.95 88.6) (stroke (width 0.1) (type solid)) (layer "Edge.Cuts"))
 (gr_arc (start 183.95 88.6) (mid 182.45 87.1) (end 183.95 85.6) (stroke (width 0.1) (type solid)) (layer "Edge.Cuts"))
 (gr_line (start 105.75 100.1) (end 113.95 100.1) (stroke (width 0.1) (type solid)) (layer "Edge.Cuts"))
 (gr_line (start 109.75 92.1) (end 105.75 92.1) (stroke (width 0.1) (type solid)) (layer "Edge.Cuts"))
 (segment (start 141.57 93.78) (end 141.1 94.25) (width 0.25) (layer "F.Cu") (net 2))
 (segment (start 141.57 92.675) (end 141.57 93.78) (width 0.25) (layer "F.Cu") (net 2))
 (segment (start 147.57 92.675) (end 147.57 94.23) (width 0.25) (layer "F.Cu") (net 2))
 (segment (start 141.07 92.675) (end 141.07 94.22) (width 0.25) (layer "F.Cu") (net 2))
 (segment (start 148.07 93.73) (end 147.55 94.25) (width 0.25) (layer "F.Cu") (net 2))
 (segment (start 148.57 93.88) (end 148.2 94.25) (width 0.25) (layer "F.Cu") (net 2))
 (segment (start 147.07 93.77) (end 147.55 94.25) (width 0.25) (layer "F.Cu") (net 2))
 (segment (start 140.57 93.72) (end 141.1 94.25) (width 0.25) (layer "F.Cu") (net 2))
 (segment (start 144.07 92.675) (end 144.07 94.03) (width 0.25) (layer "F.Cu") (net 2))
 (segment (start 139.07 94.02) (end 139.3 94.25) (width 0.25) (layer "F.Cu") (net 2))
 (segment (start 147.57 94.23) (end 147.55 94.25) (width 0.25) (layer "F.Cu") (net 2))
 (segment (start 148.57 92.675) (end 148.57 93.88) (width 0.25) (layer "F.Cu") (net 2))
 (segment (start 139.07 92.675) (end 139.07 94.02) (width 0.25) (layer "F.Cu") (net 2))
 (segment (start 139.3 94.25) (end 141.1 94.25) (width 0.25) (layer "F.Cu") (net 2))
 (segment (start 143.57 92.675) (end 143.57 93.97) (width 0.25) (layer "F.Cu") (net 2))
 (segment (start 146.85 94.25) (end 147.55 94.25) (width 0.25) (layer "F.Cu") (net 2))
 (segment (start 148.07 92.675) (end 148.07 93.73) (width 0.25) (layer "F.Cu") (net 2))
 (segment (start 143.57 93.97) (end 143.85 94.25) (width 0.25) (layer "F.Cu") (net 2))
 (segment (start 148.2 94.25) (end 147.55 94.25) (width 0.25) (layer "F.Cu") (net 2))
 (segment (start 140.57 92.675) (end 140.57 93.72) (width 0.25) (layer "F.Cu") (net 2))
 (segment (start 146.57 92.675) (end 146.57 93.97) (width 0.25) (layer "F.Cu") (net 2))
 (segment (start 147.07 92.675) (end 147.07 93.77) (width 0.25) (layer "F.Cu") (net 2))
 (segment (start 146.57 93.97) (end 146.85 94.25) (width 0.25) (layer "F.Cu") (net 2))
 (segment (start 141.07 94.22) (end 141.1 94.25) (width 0.25) (layer "F.Cu") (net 2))
 (segment (start 144.07 94.03) (end 143.85 94.25) (width 0.25) (layer "F.Cu") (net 2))
 (via (at 143.85 94.25) (size 0.8) (drill 0.4) (layers "F.Cu" "B.Cu") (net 2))
 (via (at 141.1 94.25) (size 0.8) (drill 0.4) (layers "F.Cu" "B.Cu") (free) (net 2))
 (via (at 147.55 94.25) (size 0.8) (drill 0.4) (layers "F.Cu" "B.Cu") (free) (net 2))
 (segment (start 138.07 95.17) (end 138.07 92.675) (width 0.25) (layer "F.Cu") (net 3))
 (segment (start 149.57 92.675) (end 149.57 95.18) (width 0.25) (layer "F.Cu") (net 3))
 (segment (start 149.45 95.3) (end 138.2 95.3) (width 0.25) (layer "F.Cu") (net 3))
 (segment (start 149.57 95.18) (end 149.45 95.3) (width 0.25) (layer "F.Cu") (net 3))
 (segment (start 138.2 95.3) (end 138.07 95.17) (width 0.25) (layer "F.Cu") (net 3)))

